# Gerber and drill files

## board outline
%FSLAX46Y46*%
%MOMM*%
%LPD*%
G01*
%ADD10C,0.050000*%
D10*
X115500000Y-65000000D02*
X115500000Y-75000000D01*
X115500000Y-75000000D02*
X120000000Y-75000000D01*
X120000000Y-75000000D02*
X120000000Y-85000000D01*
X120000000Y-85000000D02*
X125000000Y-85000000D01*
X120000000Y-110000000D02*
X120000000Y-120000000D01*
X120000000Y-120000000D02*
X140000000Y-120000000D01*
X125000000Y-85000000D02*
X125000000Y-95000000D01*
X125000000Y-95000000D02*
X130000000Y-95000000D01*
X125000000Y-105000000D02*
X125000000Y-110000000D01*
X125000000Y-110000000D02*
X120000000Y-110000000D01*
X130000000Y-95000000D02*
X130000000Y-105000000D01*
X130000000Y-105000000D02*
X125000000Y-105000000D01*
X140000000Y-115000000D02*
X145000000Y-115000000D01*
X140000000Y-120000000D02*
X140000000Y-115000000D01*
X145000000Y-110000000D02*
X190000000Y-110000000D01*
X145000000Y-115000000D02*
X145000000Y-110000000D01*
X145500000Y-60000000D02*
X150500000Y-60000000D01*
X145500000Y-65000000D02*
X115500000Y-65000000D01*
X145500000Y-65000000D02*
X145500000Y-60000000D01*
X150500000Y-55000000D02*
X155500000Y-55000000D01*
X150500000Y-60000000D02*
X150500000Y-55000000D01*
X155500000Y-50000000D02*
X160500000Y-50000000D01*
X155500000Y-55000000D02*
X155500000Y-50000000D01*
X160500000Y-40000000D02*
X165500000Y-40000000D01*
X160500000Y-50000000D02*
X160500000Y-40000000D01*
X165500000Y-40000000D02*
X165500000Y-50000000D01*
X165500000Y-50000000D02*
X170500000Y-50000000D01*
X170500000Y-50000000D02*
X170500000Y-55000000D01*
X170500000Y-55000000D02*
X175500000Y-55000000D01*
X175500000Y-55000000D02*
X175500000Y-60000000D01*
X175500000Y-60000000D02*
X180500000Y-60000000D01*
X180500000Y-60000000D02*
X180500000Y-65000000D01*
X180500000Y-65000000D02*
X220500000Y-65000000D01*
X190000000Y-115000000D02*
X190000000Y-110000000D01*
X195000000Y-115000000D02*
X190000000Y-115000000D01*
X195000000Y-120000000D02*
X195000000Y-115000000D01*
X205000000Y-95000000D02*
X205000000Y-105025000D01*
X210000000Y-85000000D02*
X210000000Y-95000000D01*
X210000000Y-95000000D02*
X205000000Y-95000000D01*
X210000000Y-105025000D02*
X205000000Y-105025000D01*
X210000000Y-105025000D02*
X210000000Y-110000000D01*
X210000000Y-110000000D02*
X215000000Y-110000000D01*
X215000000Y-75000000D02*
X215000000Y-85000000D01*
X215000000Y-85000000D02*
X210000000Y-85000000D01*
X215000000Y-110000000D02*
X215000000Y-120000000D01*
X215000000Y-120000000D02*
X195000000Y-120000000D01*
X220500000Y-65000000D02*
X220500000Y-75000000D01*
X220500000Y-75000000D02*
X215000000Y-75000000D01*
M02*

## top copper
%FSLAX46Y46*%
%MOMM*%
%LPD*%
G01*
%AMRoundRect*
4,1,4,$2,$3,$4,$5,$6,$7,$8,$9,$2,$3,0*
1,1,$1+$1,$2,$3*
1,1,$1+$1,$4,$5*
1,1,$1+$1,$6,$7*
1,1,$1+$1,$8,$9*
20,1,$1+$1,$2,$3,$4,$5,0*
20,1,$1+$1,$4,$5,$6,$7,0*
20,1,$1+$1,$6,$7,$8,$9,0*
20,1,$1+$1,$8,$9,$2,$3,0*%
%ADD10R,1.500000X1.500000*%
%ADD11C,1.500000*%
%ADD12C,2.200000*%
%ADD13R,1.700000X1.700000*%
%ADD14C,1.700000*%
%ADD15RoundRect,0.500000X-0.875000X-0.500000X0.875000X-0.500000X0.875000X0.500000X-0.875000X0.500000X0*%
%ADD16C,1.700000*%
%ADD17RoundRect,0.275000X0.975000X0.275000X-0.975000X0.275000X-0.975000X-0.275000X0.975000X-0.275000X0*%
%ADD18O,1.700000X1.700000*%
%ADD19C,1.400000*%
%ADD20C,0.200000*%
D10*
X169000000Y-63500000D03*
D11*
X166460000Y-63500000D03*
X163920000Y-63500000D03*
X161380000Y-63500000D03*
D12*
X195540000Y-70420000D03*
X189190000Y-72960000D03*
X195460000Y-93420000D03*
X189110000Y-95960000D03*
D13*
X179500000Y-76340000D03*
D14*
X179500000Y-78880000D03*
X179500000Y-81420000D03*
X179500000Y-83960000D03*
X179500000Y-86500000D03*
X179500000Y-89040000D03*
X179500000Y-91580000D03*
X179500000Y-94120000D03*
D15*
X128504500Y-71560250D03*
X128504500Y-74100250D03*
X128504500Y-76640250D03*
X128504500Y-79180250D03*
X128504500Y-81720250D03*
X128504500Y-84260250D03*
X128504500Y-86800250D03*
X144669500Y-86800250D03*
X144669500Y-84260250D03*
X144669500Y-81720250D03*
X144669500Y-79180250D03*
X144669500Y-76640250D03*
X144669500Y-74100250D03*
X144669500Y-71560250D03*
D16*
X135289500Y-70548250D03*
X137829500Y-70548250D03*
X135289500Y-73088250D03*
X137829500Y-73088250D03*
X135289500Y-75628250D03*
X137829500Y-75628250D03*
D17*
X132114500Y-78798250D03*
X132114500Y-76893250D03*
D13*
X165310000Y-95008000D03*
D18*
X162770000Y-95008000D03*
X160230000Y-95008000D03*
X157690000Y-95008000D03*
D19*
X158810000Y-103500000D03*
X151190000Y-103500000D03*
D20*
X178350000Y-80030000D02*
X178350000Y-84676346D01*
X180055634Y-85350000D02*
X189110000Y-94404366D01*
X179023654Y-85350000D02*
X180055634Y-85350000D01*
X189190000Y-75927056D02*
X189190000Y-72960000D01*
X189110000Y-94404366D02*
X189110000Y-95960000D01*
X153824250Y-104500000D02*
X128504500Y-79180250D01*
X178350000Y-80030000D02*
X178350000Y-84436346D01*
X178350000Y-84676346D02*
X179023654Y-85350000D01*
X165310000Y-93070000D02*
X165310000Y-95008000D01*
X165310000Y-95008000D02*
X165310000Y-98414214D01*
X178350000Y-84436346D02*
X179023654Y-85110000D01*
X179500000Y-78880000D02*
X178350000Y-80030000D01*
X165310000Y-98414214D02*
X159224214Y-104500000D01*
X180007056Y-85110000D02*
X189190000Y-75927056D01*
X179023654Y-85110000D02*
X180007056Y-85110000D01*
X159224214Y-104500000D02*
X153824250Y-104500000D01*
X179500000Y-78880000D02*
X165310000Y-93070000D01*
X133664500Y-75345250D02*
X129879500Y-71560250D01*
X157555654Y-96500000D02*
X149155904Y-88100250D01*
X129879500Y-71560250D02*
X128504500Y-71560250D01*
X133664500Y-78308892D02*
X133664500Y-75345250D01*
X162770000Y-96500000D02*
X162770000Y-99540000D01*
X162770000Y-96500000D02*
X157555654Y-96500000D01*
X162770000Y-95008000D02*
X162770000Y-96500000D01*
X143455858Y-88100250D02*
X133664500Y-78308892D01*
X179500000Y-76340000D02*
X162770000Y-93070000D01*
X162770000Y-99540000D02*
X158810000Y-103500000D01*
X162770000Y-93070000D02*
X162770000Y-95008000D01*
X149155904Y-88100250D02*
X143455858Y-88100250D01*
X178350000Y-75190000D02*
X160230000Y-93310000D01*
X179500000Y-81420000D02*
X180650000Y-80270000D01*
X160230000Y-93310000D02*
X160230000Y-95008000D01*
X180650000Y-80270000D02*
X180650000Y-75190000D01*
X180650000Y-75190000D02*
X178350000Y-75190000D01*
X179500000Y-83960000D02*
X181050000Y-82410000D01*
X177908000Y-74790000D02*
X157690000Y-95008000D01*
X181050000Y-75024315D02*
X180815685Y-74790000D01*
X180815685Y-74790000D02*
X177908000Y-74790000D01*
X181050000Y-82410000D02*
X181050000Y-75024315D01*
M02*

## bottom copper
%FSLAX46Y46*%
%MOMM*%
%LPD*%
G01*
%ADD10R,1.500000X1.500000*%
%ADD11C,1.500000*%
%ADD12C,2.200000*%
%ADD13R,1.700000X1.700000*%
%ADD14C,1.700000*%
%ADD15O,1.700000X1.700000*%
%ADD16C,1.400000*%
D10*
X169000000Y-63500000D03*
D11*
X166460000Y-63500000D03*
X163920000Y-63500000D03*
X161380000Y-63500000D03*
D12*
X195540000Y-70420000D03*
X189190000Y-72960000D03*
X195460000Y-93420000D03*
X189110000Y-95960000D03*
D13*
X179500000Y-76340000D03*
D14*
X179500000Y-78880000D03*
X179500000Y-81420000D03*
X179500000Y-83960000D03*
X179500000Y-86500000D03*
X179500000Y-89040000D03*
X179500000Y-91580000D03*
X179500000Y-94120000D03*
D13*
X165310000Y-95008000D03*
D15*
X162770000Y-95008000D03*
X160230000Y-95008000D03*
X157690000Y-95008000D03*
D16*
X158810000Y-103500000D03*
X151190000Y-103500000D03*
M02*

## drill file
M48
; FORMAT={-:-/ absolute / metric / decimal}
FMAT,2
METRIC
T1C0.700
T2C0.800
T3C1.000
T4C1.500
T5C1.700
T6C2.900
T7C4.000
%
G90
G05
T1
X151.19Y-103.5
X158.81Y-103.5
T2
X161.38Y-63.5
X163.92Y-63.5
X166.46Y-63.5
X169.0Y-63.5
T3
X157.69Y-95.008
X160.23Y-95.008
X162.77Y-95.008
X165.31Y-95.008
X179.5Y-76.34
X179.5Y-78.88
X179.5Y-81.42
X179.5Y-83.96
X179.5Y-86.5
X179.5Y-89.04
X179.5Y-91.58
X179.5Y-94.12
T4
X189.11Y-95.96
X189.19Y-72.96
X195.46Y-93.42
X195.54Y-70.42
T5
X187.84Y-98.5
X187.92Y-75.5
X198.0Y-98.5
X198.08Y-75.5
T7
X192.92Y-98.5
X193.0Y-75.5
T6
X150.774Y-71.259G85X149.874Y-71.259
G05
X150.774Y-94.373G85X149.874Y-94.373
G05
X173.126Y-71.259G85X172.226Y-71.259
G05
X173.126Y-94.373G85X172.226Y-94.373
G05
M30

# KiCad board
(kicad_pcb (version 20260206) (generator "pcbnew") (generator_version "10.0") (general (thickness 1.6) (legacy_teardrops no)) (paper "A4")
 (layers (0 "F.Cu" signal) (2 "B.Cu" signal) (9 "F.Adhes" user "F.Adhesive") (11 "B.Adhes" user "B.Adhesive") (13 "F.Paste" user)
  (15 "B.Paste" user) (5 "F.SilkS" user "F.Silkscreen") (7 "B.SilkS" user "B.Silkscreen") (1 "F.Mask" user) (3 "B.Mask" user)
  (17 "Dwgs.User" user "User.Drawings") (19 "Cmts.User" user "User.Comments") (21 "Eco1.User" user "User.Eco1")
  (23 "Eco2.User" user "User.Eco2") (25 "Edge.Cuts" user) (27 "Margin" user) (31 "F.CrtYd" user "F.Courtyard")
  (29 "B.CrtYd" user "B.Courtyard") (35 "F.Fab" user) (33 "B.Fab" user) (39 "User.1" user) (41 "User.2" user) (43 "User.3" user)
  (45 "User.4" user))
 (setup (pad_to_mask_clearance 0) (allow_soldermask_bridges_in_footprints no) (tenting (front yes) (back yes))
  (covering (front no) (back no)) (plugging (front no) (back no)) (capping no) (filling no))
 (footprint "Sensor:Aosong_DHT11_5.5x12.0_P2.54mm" (layer "F.Cu") (at 169 63.5 -90)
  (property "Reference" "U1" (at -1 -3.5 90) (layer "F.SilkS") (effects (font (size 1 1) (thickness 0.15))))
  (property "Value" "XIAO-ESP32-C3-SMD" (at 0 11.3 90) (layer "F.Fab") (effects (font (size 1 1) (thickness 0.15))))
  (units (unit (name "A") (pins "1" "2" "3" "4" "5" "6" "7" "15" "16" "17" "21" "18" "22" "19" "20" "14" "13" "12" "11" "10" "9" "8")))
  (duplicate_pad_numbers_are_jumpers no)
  (pad "1" thru_hole rect (at 0 0 270) (size 1.5 1.5) (drill 0.8) (layers "*.Cu" "*.Mask") (remove_unused_layers no)
   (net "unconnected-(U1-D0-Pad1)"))
  (pad "2" thru_hole circle (at 0 2.54 270) (size 1.5 1.5) (drill 0.8) (layers "*.Cu" "*.Mask") (remove_unused_layers no)
   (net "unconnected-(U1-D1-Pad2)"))
  (pad "3" thru_hole circle (at 0 5.08 270) (size 1.5 1.5) (drill 0.8) (layers "*.Cu" "*.Mask") (remove_unused_layers no)
   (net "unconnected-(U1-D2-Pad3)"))
  (pad "4" thru_hole circle (at 0 7.62 270) (size 1.5 1.5) (drill 0.8) (layers "*.Cu" "*.Mask") (remove_unused_layers no)
   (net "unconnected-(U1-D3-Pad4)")))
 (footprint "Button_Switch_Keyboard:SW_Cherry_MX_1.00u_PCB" (layer "F.Cu") (at 195.54 70.42)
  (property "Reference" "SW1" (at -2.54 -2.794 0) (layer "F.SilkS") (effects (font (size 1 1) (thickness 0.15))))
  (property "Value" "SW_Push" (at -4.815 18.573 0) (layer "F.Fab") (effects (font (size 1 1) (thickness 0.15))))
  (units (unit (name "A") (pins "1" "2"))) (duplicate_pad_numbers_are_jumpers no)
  (pad "" np_thru_hole circle (at -7.62 5.08) (size 1.7 1.7) (drill 1.7) (layers "*.Cu" "*.Mask"))
  (pad "" np_thru_hole circle (at -2.54 5.08) (size 4 4) (drill 4) (layers "*.Cu" "*.Mask"))
  (pad "" np_thru_hole circle (at 2.54 5.08) (size 1.7 1.7) (drill 1.7) (layers "*.Cu" "*.Mask"))
  (pad "1" thru_hole circle (at 0 0) (size 2.2 2.2) (drill 1.5) (layers "*.Cu" "*.Mask") (remove_unused_layers no) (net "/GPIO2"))
  (pad "2" thru_hole circle (at -6.35 2.54) (size 2.2 2.2) (drill 1.5) (layers "*.Cu" "*.Mask") (remove_unused_layers no) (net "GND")))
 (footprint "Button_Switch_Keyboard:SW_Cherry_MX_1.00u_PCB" (layer "F.Cu") (at 195.46 93.42)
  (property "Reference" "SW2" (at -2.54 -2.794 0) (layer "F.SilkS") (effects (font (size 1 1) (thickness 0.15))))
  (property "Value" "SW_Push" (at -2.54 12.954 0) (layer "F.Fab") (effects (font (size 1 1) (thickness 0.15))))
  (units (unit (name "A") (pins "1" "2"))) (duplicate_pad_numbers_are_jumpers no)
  (pad "" np_thru_hole circle (at -7.62 5.08) (size 1.7 1.7) (drill 1.7) (layers "*.Cu" "*.Mask"))
  (pad "" np_thru_hole circle (at -2.54 5.08) (size 4 4) (drill 4) (layers "*.Cu" "*.Mask"))
  (pad "" np_thru_hole circle (at 2.54 5.08) (size 1.7 1.7) (drill 1.7) (layers "*.Cu" "*.Mask"))
  (pad "1" thru_hole circle (at 0 0) (size 2.2 2.2) (drill 1.5) (layers "*.Cu" "*.Mask") (remove_unused_layers no) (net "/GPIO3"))
  (pad "2" thru_hole circle (at -6.35 2.54) (size 2.2 2.2) (drill 1.5) (layers "*.Cu" "*.Mask") (remove_unused_layers no) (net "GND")))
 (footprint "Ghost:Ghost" (layer "F.Cu") (at 139.5 103.5)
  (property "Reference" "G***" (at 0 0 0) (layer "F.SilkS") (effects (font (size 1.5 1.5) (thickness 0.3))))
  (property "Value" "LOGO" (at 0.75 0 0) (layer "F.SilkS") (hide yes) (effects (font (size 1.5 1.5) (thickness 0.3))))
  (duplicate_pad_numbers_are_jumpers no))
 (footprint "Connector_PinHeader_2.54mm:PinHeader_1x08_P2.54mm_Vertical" (layer "F.Cu") (at 179.5 76.34)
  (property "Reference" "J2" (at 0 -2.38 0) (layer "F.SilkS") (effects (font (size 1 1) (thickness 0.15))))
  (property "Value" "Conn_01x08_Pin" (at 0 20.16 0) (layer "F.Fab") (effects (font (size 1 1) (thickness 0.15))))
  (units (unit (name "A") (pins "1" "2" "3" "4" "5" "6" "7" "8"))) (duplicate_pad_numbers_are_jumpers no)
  (pad "1" thru_hole rect (at 0 0) (size 1.7 1.7) (drill 1) (layers "*.Cu" "*.Mask") (remove_unused_layers no) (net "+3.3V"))
  (pad "2" thru_hole circle (at 0 2.54) (size 1.7 1.7) (drill 1) (layers "*.Cu" "*.Mask") (remove_unused_layers no) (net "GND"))
  (pad "3" thru_hole circle (at 0 5.08) (size 1.7 1.7) (drill 1) (layers "*.Cu" "*.Mask") (remove_unused_layers no) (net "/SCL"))
  (pad "4" thru_hole circle (at 0 7.62) (size 1.7 1.7) (drill 1) (layers "*.Cu" "*.Mask") (remove_unused_layers no) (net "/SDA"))
  (pad "5" thru_hole circle (at 0 10.16) (size 1.7 1.7) (drill 1) (layers "*.Cu" "*.Mask") (remove_unused_layers no)
   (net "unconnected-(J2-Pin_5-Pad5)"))
  (pad "6" thru_hole circle (at 0 12.7) (size 1.7 1.7) (drill 1) (layers "*.Cu" "*.Mask") (remove_unused_layers no)
   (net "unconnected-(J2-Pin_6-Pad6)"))
  (pad "7" thru_hole circle (at 0 15.24) (size 1.7 1.7) (drill 1) (layers "*.Cu" "*.Mask") (remove_unused_layers no)
   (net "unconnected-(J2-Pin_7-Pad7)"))
  (pad "8" thru_hole circle (at 0 17.78) (size 1.7 1.7) (drill 1) (layers "*.Cu" "*.Mask") (remove_unused_layers no)
   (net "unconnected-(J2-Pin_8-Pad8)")))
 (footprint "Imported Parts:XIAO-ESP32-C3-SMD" (layer "F.Cu") (at 127.6695 89.68025)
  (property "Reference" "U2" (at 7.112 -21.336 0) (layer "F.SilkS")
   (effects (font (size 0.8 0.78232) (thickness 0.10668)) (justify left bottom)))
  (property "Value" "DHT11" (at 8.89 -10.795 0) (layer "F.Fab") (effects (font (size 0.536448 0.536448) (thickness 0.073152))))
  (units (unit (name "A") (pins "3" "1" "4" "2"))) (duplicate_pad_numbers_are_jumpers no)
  (pad "1" smd roundrect (at 0.835 -18.12) (size 2.75 2) (layers "F.Cu" "F.Mask" "F.Paste") (roundrect_rratio 0.25) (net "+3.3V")
   (solder_mask_margin 0.0508) (thermal_bridge_angle 45))
  (pad "2" smd roundrect (at 0.835 -15.58) (size 2.75 2) (layers "F.Cu" "F.Mask" "F.Paste") (roundrect_rratio 0.25) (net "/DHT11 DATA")
   (solder_mask_margin 0.0508) (thermal_bridge_angle 45))
  (pad "3" smd roundrect (at 0.835 -13.04) (size 2.75 2) (layers "F.Cu" "F.Mask" "F.Paste") (roundrect_rratio 0.25)
   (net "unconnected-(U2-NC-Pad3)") (solder_mask_margin 0.0508) (thermal_bridge_angle 45))
  (pad "4" smd roundrect (at 0.835 -10.5) (size 2.75 2) (layers "F.Cu" "F.Mask" "F.Paste") (roundrect_rratio 0.25) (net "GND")
   (solder_mask_margin 0.0508) (thermal_bridge_angle 45))
  (pad "5" smd roundrect (at 0.835 -7.96) (size 2.75 2) (layers "F.Cu" "F.Mask" "F.Paste") (roundrect_rratio 0.25)
   (solder_mask_margin 0.0508) (thermal_bridge_angle 45))
  (pad "6" smd roundrect (at 0.835 -5.42) (size 2.75 2) (layers "F.Cu" "F.Mask" "F.Paste") (roundrect_rratio 0.25)
   (solder_mask_margin 0.0508) (thermal_bridge_angle 45))
  (pad "7" smd roundrect (at 0.835 -2.88) (size 2.75 2) (layers "F.Cu" "F.Mask" "F.Paste") (roundrect_rratio 0.25)
   (solder_mask_margin 0.0508) (thermal_bridge_angle 45))
  (pad "8" smd roundrect (at 17 -2.88) (size 2.75 2) (layers "F.Cu" "F.Mask" "F.Paste") (roundrect_rratio 0.25) (solder_mask_margin 0.0508)
   (thermal_bridge_angle 45))
  (pad "9" smd roundrect (at 17 -5.42) (size 2.75 2) (layers "F.Cu" "F.Mask" "F.Paste") (roundrect_rratio 0.25) (solder_mask_margin 0.0508)
   (thermal_bridge_angle 45))
  (pad "10" smd roundrect (at 17 -7.96) (size 2.75 2) (layers "F.Cu" "F.Mask" "F.Paste") (roundrect_rratio 0.25) (solder_mask_margin 0.0508)
   (thermal_bridge_angle 45))
  (pad "11" smd roundrect (at 17 -10.5) (size 2.75 2) (layers "F.Cu" "F.Mask" "F.Paste") (roundrect_rratio 0.25) (solder_mask_margin 0.0508)
   (thermal_bridge_angle 45))
  (pad "12" smd roundrect (at 17 -13.04) (size 2.75 2) (layers "F.Cu" "F.Mask" "F.Paste") (roundrect_rratio 0.25)
   (solder_mask_margin 0.0508) (thermal_bridge_angle 45))
  (pad "13" smd roundrect (at 17 -15.58) (size 2.75 2) (layers "F.Cu" "F.Mask" "F.Paste") (roundrect_rratio 0.25)
   (solder_mask_margin 0.0508) (thermal_bridge_angle 45))
  (pad "14" smd roundrect (at 17 -18.12) (size 2.75 2) (layers "F.Cu" "F.Mask" "F.Paste") (roundrect_rratio 0.25)
   (solder_mask_margin 0.0508) (thermal_bridge_angle 45))
  (pad "15" smd circle (at 7.62 -19.132) (size 1.7 1.7) (layers "F.Cu" "F.Mask" "F.Paste"))
  (pad "16" smd circle (at 10.16 -19.132) (size 1.7 1.7) (layers "F.Cu" "F.Mask" "F.Paste"))
  (pad "17" smd circle (at 7.62 -16.592) (size 1.7 1.7) (layers "F.Cu" "F.Mask" "F.Paste"))
  (pad "18" smd circle (at 10.16 -16.592) (size 1.7 1.7) (layers "F.Cu" "F.Mask" "F.Paste"))
  (pad "19" smd circle (at 7.62 -14.052) (size 1.7 1.7) (layers "F.Cu" "F.Mask" "F.Paste"))
  (pad "20" smd circle (at 10.16 -14.052) (size 1.7 1.7) (layers "F.Cu" "F.Mask" "F.Paste"))
  (pad "21" smd roundrect (at 4.445 -10.882 180) (size 2.5 1.1) (layers "F.Cu" "F.Mask" "F.Paste") (roundrect_rratio 0.25)
   (thermal_bridge_angle 45))
  (pad "22" smd roundrect (at 4.445 -12.787 180) (size 2.5 1.1) (layers "F.Cu" "F.Mask" "F.Paste") (roundrect_rratio 0.25)
   (thermal_bridge_angle 45)))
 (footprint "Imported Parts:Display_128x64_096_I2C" (layer "F.Cu") (at 161.5 95.008 180)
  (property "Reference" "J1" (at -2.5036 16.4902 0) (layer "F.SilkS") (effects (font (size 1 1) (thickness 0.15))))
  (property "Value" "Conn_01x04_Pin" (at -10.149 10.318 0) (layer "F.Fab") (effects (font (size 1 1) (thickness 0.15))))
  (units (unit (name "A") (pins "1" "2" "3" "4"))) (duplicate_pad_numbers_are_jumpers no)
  (pad "" np_thru_hole oval (at -11.176 0.635 180) (size 3.8 2.9) (drill oval 3.8 2.9) (layers "*.Cu" "*.Mask"))
  (pad "" np_thru_hole oval (at -11.176 23.749 180) (size 3.8 2.9) (drill oval 3.8 2.9) (layers "*.Cu" "*.Mask"))
  (pad "" np_thru_hole oval (at 11.176 0.635 180) (size 3.8 2.9) (drill oval 3.8 2.9) (layers "*.Cu" "*.Mask"))
  (pad "" np_thru_hole oval (at 11.176 23.749 180) (size 3.8 2.9) (drill oval 3.8 2.9) (layers "*.Cu" "*.Mask"))
  (pad "1" thru_hole rect (at -3.81 0 270) (size 1.7 1.7) (drill 1) (layers "*.Cu" "*.Mask") (remove_unused_layers no) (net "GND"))
  (pad "2" thru_hole oval (at -1.27 0 270) (size 1.7 1.7) (drill 1) (layers "*.Cu" "*.Mask") (remove_unused_layers no) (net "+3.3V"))
  (pad "3" thru_hole oval (at 1.27 0 270) (size 1.7 1.7) (drill 1) (layers "*.Cu" "*.Mask") (remove_unused_layers no) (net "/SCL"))
  (pad "4" thru_hole oval (at 3.81 0 270) (size 1.7 1.7) (drill 1) (layers "*.Cu" "*.Mask") (remove_unused_layers no) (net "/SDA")))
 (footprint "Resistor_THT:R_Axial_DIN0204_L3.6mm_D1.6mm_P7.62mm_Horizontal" (layer "F.Cu") (at 158.81 103.5 180)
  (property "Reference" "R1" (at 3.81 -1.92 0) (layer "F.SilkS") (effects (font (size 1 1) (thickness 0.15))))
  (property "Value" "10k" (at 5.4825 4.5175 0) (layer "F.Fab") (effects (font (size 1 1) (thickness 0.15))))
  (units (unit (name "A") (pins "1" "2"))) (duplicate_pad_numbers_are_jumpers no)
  (pad "1" thru_hole circle (at 0 0 180) (size 1.4 1.4) (drill 0.7) (layers "*.Cu" "*.Mask") (remove_unused_layers no) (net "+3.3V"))
  (pad "2" thru_hole circle (at 7.62 0 180) (size 1.4 1.4) (drill 0.7) (layers "*.Cu" "*.Mask") (remove_unused_layers no)
   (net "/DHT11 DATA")))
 (gr_line (start 115.5 65) (end 115.5 75) (stroke (width 0.05) (type default)) (layer "Edge.Cuts"))
 (gr_line (start 115.5 75) (end 120 75) (stroke (width 0.05) (type default)) (layer "Edge.Cuts"))
 (gr_line (start 120 75) (end 120 85) (stroke (width 0.05) (type default)) (layer "Edge.Cuts"))
 (gr_line (start 120 85) (end 125 85) (stroke (width 0.05) (type default)) (layer "Edge.Cuts"))
 (gr_line (start 120 110) (end 120 120) (stroke (width 0.05) (type default)) (layer "Edge.Cuts"))
 (gr_line (start 120 120) (end 140 120) (stroke (width 0.05) (type default)) (layer "Edge.Cuts"))
 (gr_line (start 125 85) (end 125 95) (stroke (width 0.05) (type default)) (layer "Edge.Cuts"))
 (gr_line (start 125 95) (end 130 95) (stroke (width 0.05) (type default)) (layer "Edge.Cuts"))
 (gr_line (start 125 105) (end 125 110) (stroke (width 0.05) (type default)) (layer "Edge.Cuts"))
 (gr_line (start 125 110) (end 120 110) (stroke (width 0.05) (type default)) (layer "Edge.Cuts"))
 (gr_line (start 130 95) (end 130 105) (stroke (width 0.05) (type default)) (layer "Edge.Cuts"))
 (gr_line (start 130 105) (end 125 105) (stroke (width 0.05) (type default)) (layer "Edge.Cuts"))
 (gr_line (start 140 115) (end 145 115) (stroke (width 0.05) (type default)) (layer "Edge.Cuts"))
 (gr_line (start 140 120) (end 140 115) (stroke (width 0.05) (type default)) (layer "Edge.Cuts"))
 (gr_line (start 145 110) (end 190 110) (stroke (width 0.05) (type default)) (layer "Edge.Cuts"))
 (gr_line (start 145 115) (end 145 110) (stroke (width 0.05) (type default)) (layer "Edge.Cuts"))
 (gr_line (start 145.5 60) (end 150.5 60) (stroke (width 0.05) (type default)) (layer "Edge.Cuts"))
 (gr_line (start 145.5 65) (end 115.5 65) (stroke (width 0.05) (type default)) (layer "Edge.Cuts"))
 (gr_line (start 145.5 65) (end 145.5 60) (stroke (width 0.05) (type default)) (layer "Edge.Cuts"))
 (gr_line (start 150.5 55) (end 155.5 55) (stroke (width 0.05) (type default)) (layer "Edge.Cuts"))
 (gr_line (start 150.5 60) (end 150.5 55) (stroke (width 0.05) (type default)) (layer "Edge.Cuts"))
 (gr_line (start 155.5 50) (end 160.5 50) (stroke (width 0.05) (type default)) (layer "Edge.Cuts"))
 (gr_line (start 155.5 55) (end 155.5 50) (stroke (width 0.05) (type default)) (layer "Edge.Cuts"))
 (gr_line (start 160.5 40) (end 165.5 40) (stroke (width 0.05) (type default)) (layer "Edge.Cuts"))
 (gr_line (start 160.5 50) (end 160.5 40) (stroke (width 0.05) (type default)) (layer "Edge.Cuts"))
 (gr_line (start 165.5 40) (end 165.5 50) (stroke (width 0.05) (type default)) (layer "Edge.Cuts"))
 (gr_line (start 165.5 50) (end 170.5 50) (stroke (width 0.05) (type default)) (layer "Edge.Cuts"))
 (gr_line (start 170.5 50) (end 170.5 55) (stroke (width 0.05) (type default)) (layer "Edge.Cuts"))
 (gr_line (start 170.5 55) (end 175.5 55) (stroke (width 0.05) (type default)) (layer "Edge.Cuts"))
 (gr_line (start 175.5 55) (end 175.5 60) (stroke (width 0.05) (type default)) (layer "Edge.Cuts"))
 (gr_line (start 175.5 60) (end 180.5 60) (stroke (width 0.05) (type default)) (layer "Edge.Cuts"))
 (gr_line (start 180.5 60) (end 180.5 65) (stroke (width 0.05) (type default)) (layer "Edge.Cuts"))
 (gr_line (start 180.5 65) (end 220.5 65) (stroke (width 0.05) (type default)) (layer "Edge.Cuts"))
 (gr_line (start 190 115) (end 190 110) (stroke (width 0.05) (type default)) (layer "Edge.Cuts"))
 (gr_line (start 195 115) (end 190 115) (stroke (width 0.05) (type default)) (layer "Edge.Cuts"))
 (gr_line (start 195 120) (end 195 115) (stroke (width 0.05) (type default)) (layer "Edge.Cuts"))
 (gr_line (start 205 95) (end 205 105.025) (stroke (width 0.05) (type default)) (layer "Edge.Cuts"))
 (gr_line (start 210 85) (end 210 95) (stroke (width 0.05) (type default)) (layer "Edge.Cuts"))
 (gr_line (start 210 95) (end 205 95) (stroke (width 0.05) (type default)) (layer "Edge.Cuts"))
 (gr_line (start 210 105.025) (end 205 105.025) (stroke (width 0.05) (type default)) (layer "Edge.Cuts"))
 (gr_line (start 210 105.025) (end 210 110) (stroke (width 0.05) (type default)) (layer "Edge.Cuts"))
 (gr_line (start 210 110) (end 215 110) (stroke (width 0.05) (type default)) (layer "Edge.Cuts"))
 (gr_line (start 215 75) (end 215 85) (stroke (width 0.05) (type default)) (layer "Edge.Cuts"))
 (gr_line (start 215 85) (end 210 85) (stroke (width 0.05) (type default)) (layer "Edge.Cuts"))
 (gr_line (start 215 110) (end 215 120) (stroke (width 0.05) (type default)) (layer "Edge.Cuts"))
 (gr_line (start 215 120) (end 195 120) (stroke (width 0.05) (type default)) (layer "Edge.Cuts"))
 (gr_line (start 220.5 65) (end 220.5 75) (stroke (width 0.05) (type default)) (layer "Edge.Cuts"))
 (gr_line (start 220.5 75) (end 215 75) (stroke (width 0.05) (type default)) (layer "Edge.Cuts"))
 (segment (start 178.35 80.03) (end 178.35 84.676346) (width 0.2) (layer "F.Cu") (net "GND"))
 (segment (start 180.055634 85.35) (end 189.11 94.404366) (width 0.2) (layer "F.Cu") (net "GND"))
 (segment (start 179.023654 85.35) (end 180.055634 85.35) (width 0.2) (layer "F.Cu") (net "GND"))
 (segment (start 189.19 75.927056) (end 189.19 72.96) (width 0.2) (layer "F.Cu") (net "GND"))
 (segment (start 189.11 94.404366) (end 189.11 95.96) (width 0.2) (layer "F.Cu") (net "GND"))
 (segment (start 153.82425 104.5) (end 128.5045 79.18025) (width 0.2) (layer "F.Cu") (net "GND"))
 (segment (start 178.35 80.03) (end 178.35 84.436346) (width 0.2) (layer "F.Cu") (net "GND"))
 (segment (start 178.35 84.676346) (end 179.023654 85.35) (width 0.2) (layer "F.Cu") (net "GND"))
 (segment (start 165.31 93.07) (end 165.31 95.008) (width 0.2) (layer "F.Cu") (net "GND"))
 (segment (start 165.31 95.008) (end 165.31 98.414214) (width 0.2) (layer "F.Cu") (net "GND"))
 (segment (start 178.35 84.436346) (end 179.023654 85.11) (width 0.2) (layer "F.Cu") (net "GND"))
 (segment (start 179.5 78.88) (end 178.35 80.03) (width 0.2) (layer "F.Cu") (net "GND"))
 (segment (start 165.31 98.414214) (end 159.224214 104.5) (width 0.2) (layer "F.Cu") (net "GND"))
 (segment (start 180.007056 85.11) (end 189.19 75.927056) (width 0.2) (layer "F.Cu") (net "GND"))
 (segment (start 179.023654 85.11) (end 180.007056 85.11) (width 0.2) (layer "F.Cu") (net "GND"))
 (segment (start 159.224214 104.5) (end 153.82425 104.5) (width 0.2) (layer "F.Cu") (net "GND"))
 (segment (start 179.5 78.88) (end 165.31 93.07) (width 0.2) (layer "F.Cu") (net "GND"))
 (segment (start 133.6645 75.34525) (end 129.8795 71.56025) (width 0.2) (layer "F.Cu") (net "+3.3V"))
 (segment (start 157.555654 96.5) (end 149.155904 88.10025) (width 0.2) (layer "F.Cu") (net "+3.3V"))
 (segment (start 129.8795 71.56025) (end 128.5045 71.56025) (width 0.2) (layer "F.Cu") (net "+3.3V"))
 (segment (start 133.6645 78.308892) (end 133.6645 75.34525) (width 0.2) (layer "F.Cu") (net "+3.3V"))
 (segment (start 162.77 96.5) (end 162.77 99.54) (width 0.2) (layer "F.Cu") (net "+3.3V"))
 (segment (start 162.77 96.5) (end 157.555654 96.5) (width 0.2) (layer "F.Cu") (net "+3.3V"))
 (segment (start 162.77 95.008) (end 162.77 96.5) (width 0.2) (layer "F.Cu") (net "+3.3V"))
 (segment (start 143.455858 88.10025) (end 133.6645 78.308892) (width 0.2) (layer "F.Cu") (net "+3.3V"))
 (segment (start 179.5 76.34) (end 162.77 93.07) (width 0.2) (layer "F.Cu") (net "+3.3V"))
 (segment (start 162.77 99.54) (end 158.81 103.5) (width 0.2) (layer "F.Cu") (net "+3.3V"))
 (segment (start 162.77 93.07) (end 162.77 95.008) (width 0.2) (layer "F.Cu") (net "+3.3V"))
 (segment (start 149.155904 88.10025) (end 143.455858 88.10025) (width 0.2) (layer "F.Cu") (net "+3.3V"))
 (segment (start 178.35 75.19) (end 160.23 93.31) (width 0.2) (layer "F.Cu") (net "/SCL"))
 (segment (start 179.5 81.42) (end 180.65 80.27) (width 0.2) (layer "F.Cu") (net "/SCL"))
 (segment (start 160.23 93.31) (end 160.23 95.008) (width 0.2) (layer "F.Cu") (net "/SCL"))
 (segment (start 180.65 80.27) (end 180.65 75.19) (width 0.2) (layer "F.Cu") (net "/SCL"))
 (segment (start 180.65 75.19) (end 178.35 75.19) (width 0.2) (layer "F.Cu") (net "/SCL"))
 (segment (start 179.5 83.96) (end 181.05 82.41) (width 0.2) (layer "F.Cu") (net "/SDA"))
 (segment (start 177.908 74.79) (end 157.69 95.008) (width 0.2) (layer "F.Cu") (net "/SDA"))
 (segment (start 181.05 75.024315) (end 180.815685 74.79) (width 0.2) (layer "F.Cu") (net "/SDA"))
 (segment (start 180.815685 74.79) (end 177.908 74.79) (width 0.2) (layer "F.Cu") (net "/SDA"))
 (segment (start 181.05 82.41) (end 181.05 75.024315) (width 0.2) (layer "F.Cu") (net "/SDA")))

